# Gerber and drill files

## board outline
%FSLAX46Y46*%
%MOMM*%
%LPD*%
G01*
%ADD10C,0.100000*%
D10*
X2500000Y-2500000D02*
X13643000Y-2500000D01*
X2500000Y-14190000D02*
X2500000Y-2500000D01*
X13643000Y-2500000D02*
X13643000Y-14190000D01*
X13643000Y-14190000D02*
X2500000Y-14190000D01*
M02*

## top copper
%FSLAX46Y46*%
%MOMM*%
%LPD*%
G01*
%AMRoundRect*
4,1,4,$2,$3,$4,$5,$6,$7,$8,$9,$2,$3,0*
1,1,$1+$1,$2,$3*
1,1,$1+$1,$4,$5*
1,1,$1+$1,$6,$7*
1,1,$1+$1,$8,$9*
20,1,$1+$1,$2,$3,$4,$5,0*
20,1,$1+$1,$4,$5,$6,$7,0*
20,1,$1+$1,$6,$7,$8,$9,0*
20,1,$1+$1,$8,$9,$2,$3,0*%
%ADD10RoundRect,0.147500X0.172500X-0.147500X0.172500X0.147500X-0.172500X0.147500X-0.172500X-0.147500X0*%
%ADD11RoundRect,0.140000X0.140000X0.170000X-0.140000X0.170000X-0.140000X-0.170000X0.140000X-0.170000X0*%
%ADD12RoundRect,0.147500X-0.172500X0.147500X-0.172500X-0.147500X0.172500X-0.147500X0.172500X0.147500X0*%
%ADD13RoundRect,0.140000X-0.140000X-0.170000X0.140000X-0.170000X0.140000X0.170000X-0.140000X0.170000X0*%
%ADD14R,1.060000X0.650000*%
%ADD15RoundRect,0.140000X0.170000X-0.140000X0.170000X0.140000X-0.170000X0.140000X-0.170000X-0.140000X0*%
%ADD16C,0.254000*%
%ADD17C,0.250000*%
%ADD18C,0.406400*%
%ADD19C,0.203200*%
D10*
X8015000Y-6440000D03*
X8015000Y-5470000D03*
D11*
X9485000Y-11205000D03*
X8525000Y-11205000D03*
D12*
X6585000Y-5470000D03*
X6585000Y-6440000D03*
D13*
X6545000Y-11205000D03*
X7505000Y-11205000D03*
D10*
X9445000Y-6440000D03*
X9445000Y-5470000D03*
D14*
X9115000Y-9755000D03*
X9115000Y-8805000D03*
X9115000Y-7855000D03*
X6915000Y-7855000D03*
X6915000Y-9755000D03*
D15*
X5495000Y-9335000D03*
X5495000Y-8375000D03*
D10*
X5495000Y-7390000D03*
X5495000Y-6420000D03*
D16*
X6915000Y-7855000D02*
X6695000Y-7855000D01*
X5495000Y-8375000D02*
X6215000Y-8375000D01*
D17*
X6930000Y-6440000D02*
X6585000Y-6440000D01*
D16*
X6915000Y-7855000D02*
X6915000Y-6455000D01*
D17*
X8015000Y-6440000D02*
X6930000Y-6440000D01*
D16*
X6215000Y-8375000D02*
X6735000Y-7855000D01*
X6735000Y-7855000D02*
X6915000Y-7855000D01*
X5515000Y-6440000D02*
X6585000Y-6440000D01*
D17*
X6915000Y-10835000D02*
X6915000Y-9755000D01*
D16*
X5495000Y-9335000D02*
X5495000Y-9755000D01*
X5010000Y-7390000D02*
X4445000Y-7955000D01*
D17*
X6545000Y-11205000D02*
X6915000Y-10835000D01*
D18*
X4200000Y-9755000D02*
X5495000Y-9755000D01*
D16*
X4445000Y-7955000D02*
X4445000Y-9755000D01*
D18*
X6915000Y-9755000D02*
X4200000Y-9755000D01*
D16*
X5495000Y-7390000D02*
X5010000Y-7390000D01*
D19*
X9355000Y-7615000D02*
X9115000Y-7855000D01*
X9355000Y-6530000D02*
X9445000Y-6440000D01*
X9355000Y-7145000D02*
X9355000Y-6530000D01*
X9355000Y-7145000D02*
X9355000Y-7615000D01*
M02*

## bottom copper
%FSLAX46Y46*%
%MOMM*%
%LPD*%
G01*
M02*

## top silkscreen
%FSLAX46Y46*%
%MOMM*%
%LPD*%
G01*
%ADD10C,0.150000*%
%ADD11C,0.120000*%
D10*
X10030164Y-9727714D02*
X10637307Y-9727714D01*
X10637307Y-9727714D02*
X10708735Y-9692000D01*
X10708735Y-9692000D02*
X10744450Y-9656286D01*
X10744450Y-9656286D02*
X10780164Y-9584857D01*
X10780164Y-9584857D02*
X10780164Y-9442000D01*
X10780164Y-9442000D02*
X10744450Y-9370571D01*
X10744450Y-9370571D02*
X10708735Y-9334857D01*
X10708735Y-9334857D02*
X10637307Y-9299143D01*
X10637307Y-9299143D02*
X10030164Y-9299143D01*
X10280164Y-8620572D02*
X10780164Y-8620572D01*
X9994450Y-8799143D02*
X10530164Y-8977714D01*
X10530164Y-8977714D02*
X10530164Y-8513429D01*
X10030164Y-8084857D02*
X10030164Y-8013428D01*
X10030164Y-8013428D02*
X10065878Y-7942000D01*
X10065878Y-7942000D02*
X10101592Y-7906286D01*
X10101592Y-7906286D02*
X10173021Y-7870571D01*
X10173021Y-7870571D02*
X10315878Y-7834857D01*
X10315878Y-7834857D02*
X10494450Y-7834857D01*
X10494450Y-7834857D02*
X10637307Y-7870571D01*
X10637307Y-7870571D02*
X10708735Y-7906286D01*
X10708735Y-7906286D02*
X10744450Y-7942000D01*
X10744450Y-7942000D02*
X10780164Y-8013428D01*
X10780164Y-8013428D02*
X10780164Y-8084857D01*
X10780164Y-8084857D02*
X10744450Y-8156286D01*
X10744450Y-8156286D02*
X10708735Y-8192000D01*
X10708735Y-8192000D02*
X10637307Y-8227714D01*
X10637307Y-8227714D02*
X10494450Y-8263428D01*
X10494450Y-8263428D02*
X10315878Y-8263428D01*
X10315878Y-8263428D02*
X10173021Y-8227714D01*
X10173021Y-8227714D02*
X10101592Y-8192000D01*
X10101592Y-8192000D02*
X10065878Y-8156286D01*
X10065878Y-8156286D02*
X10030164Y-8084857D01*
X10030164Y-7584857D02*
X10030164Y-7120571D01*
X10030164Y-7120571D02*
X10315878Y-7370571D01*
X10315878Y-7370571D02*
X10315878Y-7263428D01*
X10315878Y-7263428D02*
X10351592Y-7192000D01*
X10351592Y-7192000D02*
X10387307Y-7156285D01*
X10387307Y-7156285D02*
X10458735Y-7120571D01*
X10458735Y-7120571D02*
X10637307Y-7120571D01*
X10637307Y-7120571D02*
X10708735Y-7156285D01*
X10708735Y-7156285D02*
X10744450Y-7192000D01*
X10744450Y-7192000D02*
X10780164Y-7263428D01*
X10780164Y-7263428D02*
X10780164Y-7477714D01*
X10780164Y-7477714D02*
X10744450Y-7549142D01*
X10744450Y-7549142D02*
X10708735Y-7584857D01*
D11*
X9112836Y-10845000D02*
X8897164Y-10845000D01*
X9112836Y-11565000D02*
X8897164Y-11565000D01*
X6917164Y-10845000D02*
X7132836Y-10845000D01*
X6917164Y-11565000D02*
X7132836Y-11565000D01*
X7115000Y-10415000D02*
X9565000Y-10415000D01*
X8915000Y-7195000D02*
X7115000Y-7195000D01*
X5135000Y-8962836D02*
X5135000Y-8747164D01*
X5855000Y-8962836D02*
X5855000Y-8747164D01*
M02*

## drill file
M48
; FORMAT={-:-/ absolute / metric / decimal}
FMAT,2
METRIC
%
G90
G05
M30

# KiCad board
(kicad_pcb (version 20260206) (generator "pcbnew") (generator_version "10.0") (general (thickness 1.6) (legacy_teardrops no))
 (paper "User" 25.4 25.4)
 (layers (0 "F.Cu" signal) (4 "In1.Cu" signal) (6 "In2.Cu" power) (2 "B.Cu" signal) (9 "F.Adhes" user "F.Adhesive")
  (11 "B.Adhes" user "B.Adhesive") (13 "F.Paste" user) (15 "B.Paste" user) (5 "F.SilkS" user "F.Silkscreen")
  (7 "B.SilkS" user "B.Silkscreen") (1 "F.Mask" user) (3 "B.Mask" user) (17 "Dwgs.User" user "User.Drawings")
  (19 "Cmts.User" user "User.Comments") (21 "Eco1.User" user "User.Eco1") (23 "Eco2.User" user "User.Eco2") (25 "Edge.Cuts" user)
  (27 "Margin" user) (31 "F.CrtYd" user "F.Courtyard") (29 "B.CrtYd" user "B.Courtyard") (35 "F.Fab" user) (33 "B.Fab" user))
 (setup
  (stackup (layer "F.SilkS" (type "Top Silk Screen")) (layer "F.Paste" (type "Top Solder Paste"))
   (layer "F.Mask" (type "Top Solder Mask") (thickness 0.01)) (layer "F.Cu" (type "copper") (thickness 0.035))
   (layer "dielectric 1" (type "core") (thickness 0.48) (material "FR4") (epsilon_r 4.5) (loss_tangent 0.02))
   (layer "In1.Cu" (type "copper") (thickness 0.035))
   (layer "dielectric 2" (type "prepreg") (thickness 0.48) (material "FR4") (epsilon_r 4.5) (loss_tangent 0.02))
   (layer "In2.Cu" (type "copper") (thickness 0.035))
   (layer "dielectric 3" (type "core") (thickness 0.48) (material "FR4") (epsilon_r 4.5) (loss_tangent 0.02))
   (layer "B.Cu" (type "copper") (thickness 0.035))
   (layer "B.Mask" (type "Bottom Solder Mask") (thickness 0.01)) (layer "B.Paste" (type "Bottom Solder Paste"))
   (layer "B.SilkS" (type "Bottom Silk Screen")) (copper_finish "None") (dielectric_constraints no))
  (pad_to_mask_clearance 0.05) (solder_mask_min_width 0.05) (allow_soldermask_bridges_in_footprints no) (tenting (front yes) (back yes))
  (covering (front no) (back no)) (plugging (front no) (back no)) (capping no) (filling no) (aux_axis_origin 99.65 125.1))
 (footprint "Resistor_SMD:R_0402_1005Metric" (layer "F.Cu") (at 8.015 5.955 90)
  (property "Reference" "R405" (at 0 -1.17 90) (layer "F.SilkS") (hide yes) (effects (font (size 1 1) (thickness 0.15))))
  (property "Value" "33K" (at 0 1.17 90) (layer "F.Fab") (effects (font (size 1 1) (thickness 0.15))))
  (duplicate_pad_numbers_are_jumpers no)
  (pad "1" smd roundrect (at -0.485 0 90) (size 0.59 0.64) (layers "F.Cu" "F.Mask" "F.Paste") (roundrect_rratio 0.25) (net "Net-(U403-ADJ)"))
  (pad "2" smd roundrect (at 0.485 0 90) (size 0.59 0.64) (layers "F.Cu" "F.Mask" "F.Paste") (roundrect_rratio 0.25) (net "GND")))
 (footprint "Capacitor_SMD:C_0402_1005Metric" (layer "F.Cu") (at 9.005 11.205 180)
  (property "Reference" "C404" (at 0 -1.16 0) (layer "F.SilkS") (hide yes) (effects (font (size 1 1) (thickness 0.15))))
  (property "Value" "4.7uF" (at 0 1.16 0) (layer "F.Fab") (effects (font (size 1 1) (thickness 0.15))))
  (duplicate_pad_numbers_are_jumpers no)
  (fp_line (start -0.107836 0.36) (end 0.107836 0.36) (stroke (width 0.12) (type solid)) (layer "F.SilkS"))
  (fp_line (start -0.107836 -0.36) (end 0.107836 -0.36) (stroke (width 0.12) (type solid)) (layer "F.SilkS"))
  (pad "1" smd roundrect (at -0.48 0 180) (size 0.56 0.62) (layers "F.Cu" "F.Mask" "F.Paste") (roundrect_rratio 0.25) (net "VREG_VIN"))
  (pad "2" smd roundrect (at 0.48 0 180) (size 0.56 0.62) (layers "F.Cu" "F.Mask" "F.Paste") (roundrect_rratio 0.25) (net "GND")))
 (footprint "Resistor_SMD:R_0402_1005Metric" (layer "F.Cu") (at 6.585 5.955 -90)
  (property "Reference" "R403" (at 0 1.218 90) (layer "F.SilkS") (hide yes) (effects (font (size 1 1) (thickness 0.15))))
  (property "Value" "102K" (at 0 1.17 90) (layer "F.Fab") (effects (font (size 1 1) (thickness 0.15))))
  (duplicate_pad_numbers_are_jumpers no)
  (pad "1" smd roundrect (at -0.485 0 270) (size 0.59 0.64) (layers "F.Cu" "F.Mask" "F.Paste") (roundrect_rratio 0.25) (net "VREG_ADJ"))
  (pad "2" smd roundrect (at 0.485 0 270) (size 0.59 0.64) (layers "F.Cu" "F.Mask" "F.Paste") (roundrect_rratio 0.25) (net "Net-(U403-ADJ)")))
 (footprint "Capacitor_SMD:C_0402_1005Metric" (layer "F.Cu") (at 7.025 11.205)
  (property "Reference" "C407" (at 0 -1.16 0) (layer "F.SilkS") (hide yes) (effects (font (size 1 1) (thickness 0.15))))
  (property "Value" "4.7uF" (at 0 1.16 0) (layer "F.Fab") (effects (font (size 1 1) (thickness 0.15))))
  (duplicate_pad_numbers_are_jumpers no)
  (fp_line (start -0.107836 -0.36) (end 0.107836 -0.36) (stroke (width 0.12) (type solid)) (layer "F.SilkS"))
  (fp_line (start -0.107836 0.36) (end 0.107836 0.36) (stroke (width 0.12) (type solid)) (layer "F.SilkS"))
  (pad "1" smd roundrect (at -0.48 0) (size 0.56 0.62) (layers "F.Cu" "F.Mask" "F.Paste") (roundrect_rratio 0.25) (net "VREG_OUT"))
  (pad "2" smd roundrect (at 0.48 0) (size 0.56 0.62) (layers "F.Cu" "F.Mask" "F.Paste") (roundrect_rratio 0.25) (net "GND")))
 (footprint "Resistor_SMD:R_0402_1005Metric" (layer "F.Cu") (at 9.445 5.955 90)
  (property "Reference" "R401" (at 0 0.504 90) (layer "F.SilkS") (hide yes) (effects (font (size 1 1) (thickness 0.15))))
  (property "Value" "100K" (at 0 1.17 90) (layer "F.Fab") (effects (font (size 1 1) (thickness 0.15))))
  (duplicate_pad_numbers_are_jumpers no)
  (pad "1" smd roundrect (at -0.485 0 90) (size 0.59 0.64) (layers "F.Cu" "F.Mask" "F.Paste") (roundrect_rratio 0.25) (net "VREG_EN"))
  (pad "2" smd roundrect (at 0.485 0 90) (size 0.59 0.64) (layers "F.Cu" "F.Mask" "F.Paste") (roundrect_rratio 0.25) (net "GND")))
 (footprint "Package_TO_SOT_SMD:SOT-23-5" (layer "F.Cu") (at 8.015 8.805 180)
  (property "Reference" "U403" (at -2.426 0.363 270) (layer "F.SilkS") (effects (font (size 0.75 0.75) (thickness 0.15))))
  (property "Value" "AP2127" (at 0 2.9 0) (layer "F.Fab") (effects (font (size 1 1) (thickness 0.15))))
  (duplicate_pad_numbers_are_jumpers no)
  (fp_line (start 0.9 -1.61) (end -1.55 -1.61) (stroke (width 0.12) (type solid)) (layer "F.SilkS"))
  (fp_line (start -0.9 1.61) (end 0.9 1.61) (stroke (width 0.12) (type solid)) (layer "F.SilkS"))
  (pad "1" smd rect (at -1.1 -0.95 180) (size 1.06 0.65) (layers "F.Cu" "F.Mask" "F.Paste") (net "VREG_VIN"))
  (pad "2" smd rect (at -1.1 0 180) (size 1.06 0.65) (layers "F.Cu" "F.Mask" "F.Paste") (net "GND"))
  (pad "3" smd rect (at -1.1 0.95 180) (size 1.06 0.65) (layers "F.Cu" "F.Mask" "F.Paste") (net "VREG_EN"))
  (pad "4" smd rect (at 1.1 0.95 180) (size 1.06 0.65) (layers "F.Cu" "F.Mask" "F.Paste") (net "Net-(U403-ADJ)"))
  (pad "5" smd rect (at 1.1 -0.95 180) (size 1.06 0.65) (layers "F.Cu" "F.Mask" "F.Paste") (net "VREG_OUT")))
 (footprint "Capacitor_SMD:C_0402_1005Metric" (layer "F.Cu") (at 5.495 8.855 90)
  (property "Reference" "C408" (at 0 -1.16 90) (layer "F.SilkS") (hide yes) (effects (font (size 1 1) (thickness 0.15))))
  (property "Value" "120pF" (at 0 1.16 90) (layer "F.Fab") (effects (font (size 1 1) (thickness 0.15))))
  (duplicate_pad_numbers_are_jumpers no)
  (fp_line (start -0.107836 -0.36) (end 0.107836 -0.36) (stroke (width 0.12) (type solid)) (layer "F.SilkS"))
  (fp_line (start -0.107836 0.36) (end 0.107836 0.36) (stroke (width 0.12) (type solid)) (layer "F.SilkS"))
  (pad "1" smd roundrect (at -0.48 0 90) (size 0.56 0.62) (layers "F.Cu" "F.Mask" "F.Paste") (roundrect_rratio 0.25) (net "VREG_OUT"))
  (pad "2" smd roundrect (at 0.48 0 90) (size 0.56 0.62) (layers "F.Cu" "F.Mask" "F.Paste") (roundrect_rratio 0.25) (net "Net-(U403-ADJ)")))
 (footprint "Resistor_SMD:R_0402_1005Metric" (layer "F.Cu") (at 5.495 6.905 90)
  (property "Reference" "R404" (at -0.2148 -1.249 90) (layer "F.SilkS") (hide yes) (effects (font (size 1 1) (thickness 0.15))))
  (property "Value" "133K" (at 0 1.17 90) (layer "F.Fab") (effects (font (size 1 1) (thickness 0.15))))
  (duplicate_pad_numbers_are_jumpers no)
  (pad "1" smd roundrect (at -0.485 0 90) (size 0.59 0.64) (layers "F.Cu" "F.Mask" "F.Paste") (roundrect_rratio 0.25) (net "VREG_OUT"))
  (pad "2" smd roundrect (at 0.485 0 90) (size 0.59 0.64) (layers "F.Cu" "F.Mask" "F.Paste") (roundrect_rratio 0.25) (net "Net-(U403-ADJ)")))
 (gr_line (start 2.5 2.5) (end 13.643 2.5) (stroke (width 0.1) (type default)) (layer "Edge.Cuts"))
 (gr_line (start 2.5 14.19) (end 2.5 2.5) (stroke (width 0.1) (type default)) (layer "Edge.Cuts"))
 (gr_line (start 13.643 2.5) (end 13.643 14.19) (stroke (width 0.1) (type default)) (layer "Edge.Cuts"))
 (gr_line (start 13.643 14.19) (end 2.5 14.19) (stroke (width 0.1) (type default)) (layer "Edge.Cuts"))
 (segment (start 6.915 7.855) (end 6.695 7.855) (width 0.254) (layer "F.Cu") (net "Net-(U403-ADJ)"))
 (segment (start 5.495 8.375) (end 6.215 8.375) (width 0.254) (layer "F.Cu") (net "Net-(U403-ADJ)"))
 (segment (start 6.93 6.44) (end 6.585 6.44) (width 0.25) (layer "F.Cu") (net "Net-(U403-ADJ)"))
 (segment (start 6.915 7.855) (end 6.915 6.455) (width 0.254) (layer "F.Cu") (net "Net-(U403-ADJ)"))
 (segment (start 8.015 6.44) (end 6.93 6.44) (width 0.25) (layer "F.Cu") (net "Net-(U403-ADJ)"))
 (segment (start 6.215 8.375) (end 6.735 7.855) (width 0.254) (layer "F.Cu") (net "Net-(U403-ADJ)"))
 (segment (start 6.735 7.855) (end 6.915 7.855) (width 0.254) (layer "F.Cu") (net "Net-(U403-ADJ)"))
 (segment (start 5.515 6.44) (end 6.585 6.44) (width 0.254) (layer "F.Cu") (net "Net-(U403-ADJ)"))
 (segment (start 6.915 10.835) (end 6.915 9.755) (width 0.25) (layer "F.Cu") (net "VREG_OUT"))
 (segment (start 5.495 9.335) (end 5.495 9.755) (width 0.254) (layer "F.Cu") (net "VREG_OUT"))
 (segment (start 5.01 7.39) (end 4.445 7.955) (width 0.254) (layer "F.Cu") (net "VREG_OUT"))
 (segment (start 6.545 11.205) (end 6.915 10.835) (width 0.25) (layer "F.Cu") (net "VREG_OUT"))
 (segment (start 4.2 9.755) (end 5.495 9.755) (width 0.4064) (layer "F.Cu") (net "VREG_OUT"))
 (segment (start 4.445 7.955) (end 4.445 9.755) (width 0.254) (layer "F.Cu") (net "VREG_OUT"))
 (segment (start 6.915 9.755) (end 4.2 9.755) (width 0.4064) (layer "F.Cu") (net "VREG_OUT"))
 (segment (start 5.495 7.39) (end 5.01 7.39) (width 0.254) (layer "F.Cu") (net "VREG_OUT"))
 (segment (start 9.355 7.615) (end 9.115 7.855) (width 0.2032) (layer "F.Cu") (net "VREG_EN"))
 (segment (start 9.355 6.53) (end 9.445 6.44) (width 0.2032) (layer "F.Cu") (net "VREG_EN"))
 (segment (start 9.355 7.145) (end 9.355 6.53) (width 0.2032) (layer "F.Cu") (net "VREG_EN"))
 (segment (start 9.355 7.145) (end 9.355 7.615) (width 0.2032) (layer "F.Cu") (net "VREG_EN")))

